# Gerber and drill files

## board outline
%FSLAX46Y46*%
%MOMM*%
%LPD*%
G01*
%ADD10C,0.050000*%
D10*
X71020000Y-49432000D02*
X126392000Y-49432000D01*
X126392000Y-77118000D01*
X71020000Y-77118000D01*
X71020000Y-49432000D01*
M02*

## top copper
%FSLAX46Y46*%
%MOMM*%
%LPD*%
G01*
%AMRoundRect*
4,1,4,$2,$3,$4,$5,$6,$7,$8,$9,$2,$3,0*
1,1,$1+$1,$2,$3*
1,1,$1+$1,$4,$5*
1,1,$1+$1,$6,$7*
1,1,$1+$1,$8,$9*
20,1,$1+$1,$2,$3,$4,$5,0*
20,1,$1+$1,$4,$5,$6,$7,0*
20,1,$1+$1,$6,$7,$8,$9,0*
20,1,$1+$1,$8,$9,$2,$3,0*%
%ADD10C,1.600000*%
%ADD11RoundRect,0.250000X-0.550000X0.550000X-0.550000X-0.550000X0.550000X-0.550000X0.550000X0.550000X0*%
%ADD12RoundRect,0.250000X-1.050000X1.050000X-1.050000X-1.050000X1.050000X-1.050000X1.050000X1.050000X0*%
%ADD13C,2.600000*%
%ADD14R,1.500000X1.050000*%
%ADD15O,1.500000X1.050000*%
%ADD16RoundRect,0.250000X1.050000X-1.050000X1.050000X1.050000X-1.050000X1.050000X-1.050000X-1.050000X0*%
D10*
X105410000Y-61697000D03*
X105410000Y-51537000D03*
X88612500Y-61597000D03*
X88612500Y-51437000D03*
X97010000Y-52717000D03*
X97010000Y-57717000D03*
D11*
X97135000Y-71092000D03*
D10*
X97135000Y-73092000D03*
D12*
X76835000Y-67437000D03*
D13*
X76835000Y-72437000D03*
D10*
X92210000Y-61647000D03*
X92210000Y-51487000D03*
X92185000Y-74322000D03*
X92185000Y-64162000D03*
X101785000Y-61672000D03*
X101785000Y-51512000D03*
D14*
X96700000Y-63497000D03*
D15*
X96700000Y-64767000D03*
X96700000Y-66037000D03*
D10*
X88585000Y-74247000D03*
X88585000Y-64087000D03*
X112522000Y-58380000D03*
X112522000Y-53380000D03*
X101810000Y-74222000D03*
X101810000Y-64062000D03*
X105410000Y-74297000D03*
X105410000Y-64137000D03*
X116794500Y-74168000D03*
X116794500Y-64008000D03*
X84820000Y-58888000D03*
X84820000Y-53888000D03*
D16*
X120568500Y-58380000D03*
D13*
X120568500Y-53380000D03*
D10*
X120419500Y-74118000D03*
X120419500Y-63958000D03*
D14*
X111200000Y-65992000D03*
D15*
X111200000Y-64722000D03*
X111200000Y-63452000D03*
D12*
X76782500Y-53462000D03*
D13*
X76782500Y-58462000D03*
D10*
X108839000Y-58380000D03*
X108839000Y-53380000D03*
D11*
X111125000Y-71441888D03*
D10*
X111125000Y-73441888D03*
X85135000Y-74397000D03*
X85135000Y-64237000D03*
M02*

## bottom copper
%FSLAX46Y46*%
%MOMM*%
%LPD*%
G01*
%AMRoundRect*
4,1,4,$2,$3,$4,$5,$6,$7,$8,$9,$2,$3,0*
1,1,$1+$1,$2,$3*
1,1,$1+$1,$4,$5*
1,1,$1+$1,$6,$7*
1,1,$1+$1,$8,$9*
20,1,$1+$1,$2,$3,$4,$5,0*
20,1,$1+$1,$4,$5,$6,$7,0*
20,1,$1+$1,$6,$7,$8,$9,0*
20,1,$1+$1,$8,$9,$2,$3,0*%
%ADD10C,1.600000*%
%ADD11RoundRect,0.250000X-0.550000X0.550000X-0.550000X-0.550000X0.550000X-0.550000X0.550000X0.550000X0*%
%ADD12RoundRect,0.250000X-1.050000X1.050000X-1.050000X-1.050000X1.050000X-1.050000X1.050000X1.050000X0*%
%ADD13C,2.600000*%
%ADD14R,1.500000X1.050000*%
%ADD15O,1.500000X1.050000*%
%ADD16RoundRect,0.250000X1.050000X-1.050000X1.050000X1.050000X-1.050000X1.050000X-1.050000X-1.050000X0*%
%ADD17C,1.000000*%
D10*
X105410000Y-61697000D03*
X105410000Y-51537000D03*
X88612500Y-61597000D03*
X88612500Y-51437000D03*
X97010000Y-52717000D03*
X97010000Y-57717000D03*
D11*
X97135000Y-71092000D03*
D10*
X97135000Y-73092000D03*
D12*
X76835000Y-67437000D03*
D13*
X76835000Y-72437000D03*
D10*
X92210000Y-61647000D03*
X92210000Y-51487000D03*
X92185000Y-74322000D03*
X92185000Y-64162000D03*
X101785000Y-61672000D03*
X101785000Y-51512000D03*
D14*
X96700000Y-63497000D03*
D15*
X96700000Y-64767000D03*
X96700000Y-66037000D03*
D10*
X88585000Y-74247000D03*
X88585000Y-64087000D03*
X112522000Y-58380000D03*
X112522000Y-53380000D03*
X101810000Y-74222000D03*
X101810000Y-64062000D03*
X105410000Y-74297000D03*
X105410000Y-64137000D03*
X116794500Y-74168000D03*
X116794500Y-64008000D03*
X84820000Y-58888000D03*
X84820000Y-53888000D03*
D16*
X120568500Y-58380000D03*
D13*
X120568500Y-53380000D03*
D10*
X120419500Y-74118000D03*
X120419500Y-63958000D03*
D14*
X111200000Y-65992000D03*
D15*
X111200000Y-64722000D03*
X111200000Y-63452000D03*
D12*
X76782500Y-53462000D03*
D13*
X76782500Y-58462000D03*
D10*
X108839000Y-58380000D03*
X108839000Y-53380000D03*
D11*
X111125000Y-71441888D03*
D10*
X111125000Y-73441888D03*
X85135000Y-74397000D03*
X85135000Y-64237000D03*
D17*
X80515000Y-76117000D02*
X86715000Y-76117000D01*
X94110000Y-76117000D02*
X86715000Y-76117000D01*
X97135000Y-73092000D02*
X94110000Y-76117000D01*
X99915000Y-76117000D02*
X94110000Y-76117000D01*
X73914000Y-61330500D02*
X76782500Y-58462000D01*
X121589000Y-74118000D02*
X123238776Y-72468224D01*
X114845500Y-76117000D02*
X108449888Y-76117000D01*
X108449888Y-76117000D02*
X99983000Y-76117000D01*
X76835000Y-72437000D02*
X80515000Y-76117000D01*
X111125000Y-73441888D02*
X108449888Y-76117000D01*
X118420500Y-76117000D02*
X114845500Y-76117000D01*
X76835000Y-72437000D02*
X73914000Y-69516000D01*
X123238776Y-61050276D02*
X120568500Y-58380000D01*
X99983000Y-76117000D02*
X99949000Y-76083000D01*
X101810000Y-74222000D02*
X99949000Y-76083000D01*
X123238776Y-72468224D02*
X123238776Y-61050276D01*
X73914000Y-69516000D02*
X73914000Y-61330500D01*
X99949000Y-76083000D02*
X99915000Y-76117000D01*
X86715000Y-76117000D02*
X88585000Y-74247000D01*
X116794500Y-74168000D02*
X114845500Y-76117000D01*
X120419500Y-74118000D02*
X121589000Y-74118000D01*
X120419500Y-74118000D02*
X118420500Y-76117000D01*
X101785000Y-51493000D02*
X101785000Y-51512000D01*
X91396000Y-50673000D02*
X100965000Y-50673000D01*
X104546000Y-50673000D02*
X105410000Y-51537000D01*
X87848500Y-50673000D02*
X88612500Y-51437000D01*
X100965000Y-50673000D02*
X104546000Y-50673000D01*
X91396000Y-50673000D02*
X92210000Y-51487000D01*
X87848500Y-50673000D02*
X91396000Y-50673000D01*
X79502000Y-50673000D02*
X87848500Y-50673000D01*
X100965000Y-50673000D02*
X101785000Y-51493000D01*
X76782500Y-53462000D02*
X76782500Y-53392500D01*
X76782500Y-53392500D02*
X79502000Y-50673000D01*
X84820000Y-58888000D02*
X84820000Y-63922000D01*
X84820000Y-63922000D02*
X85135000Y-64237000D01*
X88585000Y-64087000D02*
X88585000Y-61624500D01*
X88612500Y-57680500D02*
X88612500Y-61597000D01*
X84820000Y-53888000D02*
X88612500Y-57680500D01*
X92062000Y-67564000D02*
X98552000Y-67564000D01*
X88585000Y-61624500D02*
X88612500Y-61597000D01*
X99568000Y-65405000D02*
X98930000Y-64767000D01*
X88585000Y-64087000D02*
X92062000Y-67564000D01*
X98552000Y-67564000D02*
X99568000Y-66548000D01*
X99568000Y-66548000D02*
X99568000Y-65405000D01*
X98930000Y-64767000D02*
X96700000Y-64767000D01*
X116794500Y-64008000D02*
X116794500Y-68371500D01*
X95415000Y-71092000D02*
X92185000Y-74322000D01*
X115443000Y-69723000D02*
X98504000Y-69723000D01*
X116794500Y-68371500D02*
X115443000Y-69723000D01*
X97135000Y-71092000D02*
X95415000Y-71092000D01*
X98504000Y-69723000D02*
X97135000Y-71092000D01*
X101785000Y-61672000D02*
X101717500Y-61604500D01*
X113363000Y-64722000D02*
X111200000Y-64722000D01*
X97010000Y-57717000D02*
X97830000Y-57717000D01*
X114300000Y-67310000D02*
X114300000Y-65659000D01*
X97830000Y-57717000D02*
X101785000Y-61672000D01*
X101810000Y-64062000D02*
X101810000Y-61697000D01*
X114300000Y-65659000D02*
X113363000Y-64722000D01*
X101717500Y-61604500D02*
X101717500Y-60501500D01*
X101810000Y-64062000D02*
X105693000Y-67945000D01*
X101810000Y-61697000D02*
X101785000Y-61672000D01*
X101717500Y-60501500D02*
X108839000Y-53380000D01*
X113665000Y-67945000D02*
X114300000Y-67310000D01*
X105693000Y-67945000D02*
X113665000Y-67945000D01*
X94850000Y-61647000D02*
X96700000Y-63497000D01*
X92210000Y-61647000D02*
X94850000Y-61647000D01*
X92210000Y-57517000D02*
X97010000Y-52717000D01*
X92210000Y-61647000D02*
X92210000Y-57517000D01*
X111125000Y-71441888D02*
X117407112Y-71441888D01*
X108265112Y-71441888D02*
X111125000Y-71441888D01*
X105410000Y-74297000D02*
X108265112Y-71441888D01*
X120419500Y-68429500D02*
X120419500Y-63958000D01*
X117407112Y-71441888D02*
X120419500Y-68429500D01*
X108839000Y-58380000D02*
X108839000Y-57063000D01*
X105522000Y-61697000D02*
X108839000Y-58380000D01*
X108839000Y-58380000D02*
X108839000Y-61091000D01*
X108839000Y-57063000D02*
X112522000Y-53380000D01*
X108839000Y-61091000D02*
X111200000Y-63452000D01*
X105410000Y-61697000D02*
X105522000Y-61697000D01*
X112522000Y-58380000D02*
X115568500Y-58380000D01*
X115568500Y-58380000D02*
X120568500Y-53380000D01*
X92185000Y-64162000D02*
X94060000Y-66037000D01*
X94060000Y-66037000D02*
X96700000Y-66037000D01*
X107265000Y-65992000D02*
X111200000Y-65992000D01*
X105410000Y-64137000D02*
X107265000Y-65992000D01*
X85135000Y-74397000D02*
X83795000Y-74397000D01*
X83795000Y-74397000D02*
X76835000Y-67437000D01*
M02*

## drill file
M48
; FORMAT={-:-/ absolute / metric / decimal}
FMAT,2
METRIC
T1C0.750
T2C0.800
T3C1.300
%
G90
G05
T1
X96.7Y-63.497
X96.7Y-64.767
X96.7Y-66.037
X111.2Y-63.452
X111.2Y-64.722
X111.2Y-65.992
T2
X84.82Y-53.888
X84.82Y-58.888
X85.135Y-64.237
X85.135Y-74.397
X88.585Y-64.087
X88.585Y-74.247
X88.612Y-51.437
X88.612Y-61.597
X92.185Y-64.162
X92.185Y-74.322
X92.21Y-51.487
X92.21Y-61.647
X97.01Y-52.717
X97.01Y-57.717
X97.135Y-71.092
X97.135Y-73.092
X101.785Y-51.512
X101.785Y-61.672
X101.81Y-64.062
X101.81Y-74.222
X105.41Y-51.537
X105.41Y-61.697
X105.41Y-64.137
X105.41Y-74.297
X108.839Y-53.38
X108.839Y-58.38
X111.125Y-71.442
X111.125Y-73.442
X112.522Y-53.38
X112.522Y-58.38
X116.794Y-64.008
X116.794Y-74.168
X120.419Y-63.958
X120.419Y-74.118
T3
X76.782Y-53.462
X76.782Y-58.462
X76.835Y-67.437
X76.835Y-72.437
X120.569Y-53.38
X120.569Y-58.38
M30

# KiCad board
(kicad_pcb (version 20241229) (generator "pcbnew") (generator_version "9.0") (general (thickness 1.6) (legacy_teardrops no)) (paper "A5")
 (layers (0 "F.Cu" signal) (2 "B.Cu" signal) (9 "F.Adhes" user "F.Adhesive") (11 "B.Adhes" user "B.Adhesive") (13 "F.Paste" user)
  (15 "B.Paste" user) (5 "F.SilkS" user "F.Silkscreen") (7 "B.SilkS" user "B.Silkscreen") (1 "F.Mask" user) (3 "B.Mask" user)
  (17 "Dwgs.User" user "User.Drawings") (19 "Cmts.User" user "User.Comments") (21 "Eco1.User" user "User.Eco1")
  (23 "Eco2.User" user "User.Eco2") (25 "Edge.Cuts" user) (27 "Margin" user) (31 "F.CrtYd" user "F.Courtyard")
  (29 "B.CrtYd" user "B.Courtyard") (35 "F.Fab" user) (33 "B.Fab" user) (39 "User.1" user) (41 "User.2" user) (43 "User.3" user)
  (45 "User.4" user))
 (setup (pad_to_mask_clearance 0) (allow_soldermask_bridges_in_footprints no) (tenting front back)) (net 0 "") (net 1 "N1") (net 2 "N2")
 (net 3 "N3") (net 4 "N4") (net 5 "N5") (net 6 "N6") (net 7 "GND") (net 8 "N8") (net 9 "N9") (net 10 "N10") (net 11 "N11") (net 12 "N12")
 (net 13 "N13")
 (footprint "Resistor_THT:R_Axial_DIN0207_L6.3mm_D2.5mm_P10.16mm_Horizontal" (layer "F.Cu") (at 105.41 61.697 90)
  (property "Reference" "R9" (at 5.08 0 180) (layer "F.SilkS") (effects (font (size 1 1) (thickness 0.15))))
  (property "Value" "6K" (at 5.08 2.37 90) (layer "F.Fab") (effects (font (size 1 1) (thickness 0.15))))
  (pad "1" thru_hole circle (at 0 0 90) (size 1.6 1.6) (drill 0.8) (layers "*.Cu" "*.Mask") (remove_unused_layers no) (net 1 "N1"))
  (pad "2" thru_hole circle (at 10.16 0 90) (size 1.6 1.6) (drill 0.8) (layers "*.Cu" "*.Mask") (remove_unused_layers no) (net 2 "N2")))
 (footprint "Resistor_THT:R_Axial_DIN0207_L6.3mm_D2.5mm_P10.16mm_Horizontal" (layer "F.Cu") (at 88.6125 61.597 90)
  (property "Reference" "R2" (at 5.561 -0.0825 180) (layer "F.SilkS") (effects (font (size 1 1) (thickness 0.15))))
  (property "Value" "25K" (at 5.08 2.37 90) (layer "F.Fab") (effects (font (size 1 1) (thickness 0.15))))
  (pad "1" thru_hole circle (at 0 0 90) (size 1.6 1.6) (drill 0.8) (layers "*.Cu" "*.Mask") (remove_unused_layers no) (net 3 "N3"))
  (pad "2" thru_hole circle (at 10.16 0 90) (size 1.6 1.6) (drill 0.8) (layers "*.Cu" "*.Mask") (remove_unused_layers no) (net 2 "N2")))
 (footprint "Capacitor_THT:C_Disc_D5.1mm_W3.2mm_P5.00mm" (layer "F.Cu") (at 97.01 52.717 -90)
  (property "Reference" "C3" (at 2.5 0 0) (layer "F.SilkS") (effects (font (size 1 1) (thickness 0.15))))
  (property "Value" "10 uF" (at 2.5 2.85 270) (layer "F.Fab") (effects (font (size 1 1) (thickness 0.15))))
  (pad "1" thru_hole circle (at 0 0 270) (size 1.6 1.6) (drill 0.8) (layers "*.Cu" "*.Mask") (remove_unused_layers no) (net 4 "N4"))
  (pad "2" thru_hole circle (at 5 0 270) (size 1.6 1.6) (drill 0.8) (layers "*.Cu" "*.Mask") (remove_unused_layers no) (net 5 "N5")))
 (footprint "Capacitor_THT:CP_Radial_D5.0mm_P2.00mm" (layer "F.Cu") (at 97.135 71.092 -90)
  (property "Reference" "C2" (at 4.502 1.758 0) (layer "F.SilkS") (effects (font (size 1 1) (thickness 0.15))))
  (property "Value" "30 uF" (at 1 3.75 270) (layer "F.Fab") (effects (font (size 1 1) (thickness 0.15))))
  (pad "1" thru_hole roundrect (at 0 0 270) (size 1.6 1.6) (drill 0.8) (layers "*.Cu" "*.Mask") (remove_unused_layers no)
   (roundrect_rratio 0.15625) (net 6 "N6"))
  (pad "2" thru_hole circle (at 2 0 270) (size 1.6 1.6) (drill 0.8) (layers "*.Cu" "*.Mask") (remove_unused_layers no) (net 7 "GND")))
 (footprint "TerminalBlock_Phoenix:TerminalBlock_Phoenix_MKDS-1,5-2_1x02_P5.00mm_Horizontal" (layer "F.Cu") (at 76.835 67.437 -90)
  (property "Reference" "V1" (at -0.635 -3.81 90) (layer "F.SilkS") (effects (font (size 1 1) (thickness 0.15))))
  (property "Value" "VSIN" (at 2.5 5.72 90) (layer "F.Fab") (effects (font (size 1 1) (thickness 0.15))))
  (pad "1" thru_hole roundrect (at 0 0 270) (size 2.6 2.6) (drill 1.3) (layers "*.Cu" "*.Mask") (remove_unused_layers no)
   (roundrect_rratio 0.096154) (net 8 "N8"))
  (pad "2" thru_hole circle (at 5 0 270) (size 2.6 2.6) (drill 1.3) (layers "*.Cu" "*.Mask") (remove_unused_layers no) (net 7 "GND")))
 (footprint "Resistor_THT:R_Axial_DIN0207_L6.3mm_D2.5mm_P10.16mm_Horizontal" (layer "F.Cu") (at 92.21 61.647 90)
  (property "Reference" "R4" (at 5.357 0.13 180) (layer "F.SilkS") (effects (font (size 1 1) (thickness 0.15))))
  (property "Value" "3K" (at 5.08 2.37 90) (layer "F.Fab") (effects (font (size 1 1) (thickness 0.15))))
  (pad "1" thru_hole circle (at 0 0 90) (size 1.6 1.6) (drill 0.8) (layers "*.Cu" "*.Mask") (remove_unused_layers no) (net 4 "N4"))
  (pad "2" thru_hole circle (at 10.16 0 90) (size 1.6 1.6) (drill 0.8) (layers "*.Cu" "*.Mask") (remove_unused_layers no) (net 2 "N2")))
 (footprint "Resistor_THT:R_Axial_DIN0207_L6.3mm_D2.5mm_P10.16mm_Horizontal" (layer "F.Cu") (at 92.185 74.322 90)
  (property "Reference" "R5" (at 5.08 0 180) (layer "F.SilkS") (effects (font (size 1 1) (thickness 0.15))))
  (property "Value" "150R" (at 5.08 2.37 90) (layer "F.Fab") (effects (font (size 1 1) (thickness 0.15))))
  (pad "1" thru_hole circle (at 0 0 90) (size 1.6 1.6) (drill 0.8) (layers "*.Cu" "*.Mask") (remove_unused_layers no) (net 6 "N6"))
  (pad "2" thru_hole circle (at 10.16 0 90) (size 1.6 1.6) (drill 0.8) (layers "*.Cu" "*.Mask") (remove_unused_layers no) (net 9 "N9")))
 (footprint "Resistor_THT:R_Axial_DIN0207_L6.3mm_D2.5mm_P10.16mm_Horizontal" (layer "F.Cu") (at 101.785 61.672 90)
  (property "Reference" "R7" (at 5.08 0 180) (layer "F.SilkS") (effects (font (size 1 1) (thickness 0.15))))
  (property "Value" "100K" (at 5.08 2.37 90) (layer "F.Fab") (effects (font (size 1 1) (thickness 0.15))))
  (pad "1" thru_hole circle (at 0 0 90) (size 1.6 1.6) (drill 0.8) (layers "*.Cu" "*.Mask") (remove_unused_layers no) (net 5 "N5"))
  (pad "2" thru_hole circle (at 10.16 0 90) (size 1.6 1.6) (drill 0.8) (layers "*.Cu" "*.Mask") (remove_unused_layers no) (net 2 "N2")))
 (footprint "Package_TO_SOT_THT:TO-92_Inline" (layer "F.Cu") (at 96.7 63.497 -90)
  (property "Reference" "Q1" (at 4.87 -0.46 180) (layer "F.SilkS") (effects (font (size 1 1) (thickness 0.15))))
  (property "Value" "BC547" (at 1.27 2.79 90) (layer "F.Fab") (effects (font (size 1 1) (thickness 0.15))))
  (pad "1" thru_hole rect (at 0 0 270) (size 1.05 1.5) (drill 0.75) (layers "*.Cu" "*.Mask") (remove_unused_layers no) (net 4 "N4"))
  (pad "2" thru_hole oval (at 1.27 0 270) (size 1.05 1.5) (drill 0.75) (layers "*.Cu" "*.Mask") (remove_unused_layers no) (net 3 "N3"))
  (pad "3" thru_hole oval (at 2.54 0 270) (size 1.05 1.5) (drill 0.75) (layers "*.Cu" "*.Mask") (remove_unused_layers no) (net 9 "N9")))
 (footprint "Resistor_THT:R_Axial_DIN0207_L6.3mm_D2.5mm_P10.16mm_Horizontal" (layer "F.Cu") (at 88.585 74.247 90)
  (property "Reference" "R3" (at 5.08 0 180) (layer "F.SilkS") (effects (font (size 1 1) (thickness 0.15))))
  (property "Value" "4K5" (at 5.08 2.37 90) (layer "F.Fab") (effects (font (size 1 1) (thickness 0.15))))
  (pad "1" thru_hole circle (at 0 0 90) (size 1.6 1.6) (drill 0.8) (layers "*.Cu" "*.Mask") (remove_unused_layers no) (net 7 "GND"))
  (pad "2" thru_hole circle (at 10.16 0 90) (size 1.6 1.6) (drill 0.8) (layers "*.Cu" "*.Mask") (remove_unused_layers no) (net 3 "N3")))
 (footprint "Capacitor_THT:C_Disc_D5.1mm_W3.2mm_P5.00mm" (layer "F.Cu") (at 112.522 58.38 90)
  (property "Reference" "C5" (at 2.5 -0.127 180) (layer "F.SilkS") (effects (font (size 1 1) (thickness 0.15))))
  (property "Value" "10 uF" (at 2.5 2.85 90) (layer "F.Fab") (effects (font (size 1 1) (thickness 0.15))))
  (pad "1" thru_hole circle (at 0 0 90) (size 1.6 1.6) (drill 0.8) (layers "*.Cu" "*.Mask") (remove_unused_layers no) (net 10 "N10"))
  (pad "2" thru_hole circle (at 5 0 90) (size 1.6 1.6) (drill 0.8) (layers "*.Cu" "*.Mask") (remove_unused_layers no) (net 1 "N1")))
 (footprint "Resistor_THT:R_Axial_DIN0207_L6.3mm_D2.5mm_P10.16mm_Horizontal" (layer "F.Cu") (at 101.81 74.222 90)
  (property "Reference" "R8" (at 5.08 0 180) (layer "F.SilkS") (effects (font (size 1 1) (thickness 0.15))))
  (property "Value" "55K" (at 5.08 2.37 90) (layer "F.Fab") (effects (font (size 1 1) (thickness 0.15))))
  (pad "1" thru_hole circle (at 0 0 90) (size 1.6 1.6) (drill 0.8) (layers "*.Cu" "*.Mask") (remove_unused_layers no) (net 7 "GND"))
  (pad "2" thru_hole circle (at 10.16 0 90) (size 1.6 1.6) (drill 0.8) (layers "*.Cu" "*.Mask") (remove_unused_layers no) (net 5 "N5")))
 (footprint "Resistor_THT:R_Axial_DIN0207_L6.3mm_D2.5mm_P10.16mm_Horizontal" (layer "F.Cu") (at 105.41 74.297 90)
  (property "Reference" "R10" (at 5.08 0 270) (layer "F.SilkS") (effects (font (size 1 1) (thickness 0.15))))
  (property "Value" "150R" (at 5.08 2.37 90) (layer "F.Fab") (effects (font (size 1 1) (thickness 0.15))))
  (pad "1" thru_hole circle (at 0 0 90) (size 1.6 1.6) (drill 0.8) (layers "*.Cu" "*.Mask") (remove_unused_layers no) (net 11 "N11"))
  (pad "2" thru_hole circle (at 10.16 0 90) (size 1.6 1.6) (drill 0.8) (layers "*.Cu" "*.Mask") (remove_unused_layers no) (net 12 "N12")))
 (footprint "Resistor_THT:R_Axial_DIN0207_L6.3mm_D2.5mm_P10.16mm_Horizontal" (layer "F.Cu") (at 116.7945 74.168 90)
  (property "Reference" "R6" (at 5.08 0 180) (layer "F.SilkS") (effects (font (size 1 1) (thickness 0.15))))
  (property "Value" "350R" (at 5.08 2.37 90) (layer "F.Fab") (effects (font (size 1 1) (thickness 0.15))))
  (pad "1" thru_hole circle (at 0 0 90) (size 1.6 1.6) (drill 0.8) (layers "*.Cu" "*.Mask") (remove_unused_layers no) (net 7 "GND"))
  (pad "2" thru_hole circle (at 10.16 0 90) (size 1.6 1.6) (drill 0.8) (layers "*.Cu" "*.Mask") (remove_unused_layers no) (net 6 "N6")))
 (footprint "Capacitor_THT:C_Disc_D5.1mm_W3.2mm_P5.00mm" (layer "F.Cu") (at 84.82 58.888 90)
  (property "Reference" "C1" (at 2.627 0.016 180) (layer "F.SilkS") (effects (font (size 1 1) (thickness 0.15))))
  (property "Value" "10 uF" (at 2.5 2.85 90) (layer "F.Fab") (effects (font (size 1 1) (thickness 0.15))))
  (pad "1" thru_hole circle (at 0 0 90) (size 1.6 1.6) (drill 0.8) (layers "*.Cu" "*.Mask") (remove_unused_layers no) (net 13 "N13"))
  (pad "2" thru_hole circle (at 5 0 90) (size 1.6 1.6) (drill 0.8) (layers "*.Cu" "*.Mask") (remove_unused_layers no) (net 3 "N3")))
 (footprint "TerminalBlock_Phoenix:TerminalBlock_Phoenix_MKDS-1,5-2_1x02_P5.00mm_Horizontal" (layer "F.Cu") (at 120.5685 58.38 90)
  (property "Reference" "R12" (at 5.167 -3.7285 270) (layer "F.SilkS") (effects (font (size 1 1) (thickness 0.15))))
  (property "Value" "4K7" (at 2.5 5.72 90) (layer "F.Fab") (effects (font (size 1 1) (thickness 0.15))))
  (pad "1" thru_hole roundrect (at 0 0 90) (size 2.6 2.6) (drill 1.3) (layers "*.Cu" "*.Mask") (remove_unused_layers no)
   (roundrect_rratio 0.096154) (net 7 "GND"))
  (pad "2" thru_hole circle (at 5 0 90) (size 2.6 2.6) (drill 1.3) (layers "*.Cu" "*.Mask") (remove_unused_layers no) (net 10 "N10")))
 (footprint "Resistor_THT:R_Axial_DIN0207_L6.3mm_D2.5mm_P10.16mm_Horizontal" (layer "F.Cu") (at 120.4195 74.118 90)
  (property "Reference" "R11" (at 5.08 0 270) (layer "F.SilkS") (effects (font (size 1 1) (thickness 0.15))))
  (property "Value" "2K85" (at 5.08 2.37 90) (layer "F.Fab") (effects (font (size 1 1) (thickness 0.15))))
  (pad "1" thru_hole circle (at 0 0 90) (size 1.6 1.6) (drill 0.8) (layers "*.Cu" "*.Mask") (remove_unused_layers no) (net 7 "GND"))
  (pad "2" thru_hole circle (at 10.16 0 90) (size 1.6 1.6) (drill 0.8) (layers "*.Cu" "*.Mask") (remove_unused_layers no) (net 11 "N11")))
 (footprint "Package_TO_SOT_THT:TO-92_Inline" (layer "F.Cu") (at 111.2 65.992 90)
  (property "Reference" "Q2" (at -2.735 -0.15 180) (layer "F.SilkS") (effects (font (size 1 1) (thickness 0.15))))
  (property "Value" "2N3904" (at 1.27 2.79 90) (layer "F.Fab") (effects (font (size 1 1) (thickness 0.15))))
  (pad "1" thru_hole rect (at 0 0 90) (size 1.05 1.5) (drill 0.75) (layers "*.Cu" "*.Mask") (remove_unused_layers no) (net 12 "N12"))
  (pad "2" thru_hole oval (at 1.27 0 90) (size 1.05 1.5) (drill 0.75) (layers "*.Cu" "*.Mask") (remove_unused_layers no) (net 5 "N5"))
  (pad "3" thru_hole oval (at 2.54 0 90) (size 1.05 1.5) (drill 0.75) (layers "*.Cu" "*.Mask") (remove_unused_layers no) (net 1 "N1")))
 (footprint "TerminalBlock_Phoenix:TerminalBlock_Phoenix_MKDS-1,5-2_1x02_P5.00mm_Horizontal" (layer "F.Cu") (at 76.7825 53.462 -90)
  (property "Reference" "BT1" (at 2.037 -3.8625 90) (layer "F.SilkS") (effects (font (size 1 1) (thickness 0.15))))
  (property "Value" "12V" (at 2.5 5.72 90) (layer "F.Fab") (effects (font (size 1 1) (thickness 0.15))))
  (pad "1" thru_hole roundrect (at 0 0 270) (size 2.6 2.6) (drill 1.3) (layers "*.Cu" "*.Mask") (remove_unused_layers no)
   (roundrect_rratio 0.096154) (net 2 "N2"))
  (pad "2" thru_hole circle (at 5 0 270) (size 2.6 2.6) (drill 1.3) (layers "*.Cu" "*.Mask") (remove_unused_layers no) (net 7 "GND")))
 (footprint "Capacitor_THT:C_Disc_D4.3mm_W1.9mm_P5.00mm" (layer "F.Cu") (at 108.839 58.38 90)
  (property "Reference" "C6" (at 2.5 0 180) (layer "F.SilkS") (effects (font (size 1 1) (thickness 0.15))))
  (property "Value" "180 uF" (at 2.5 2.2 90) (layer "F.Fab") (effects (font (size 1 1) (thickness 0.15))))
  (pad "1" thru_hole circle (at 0 0 90) (size 1.6 1.6) (drill 0.8) (layers "*.Cu" "*.Mask") (remove_unused_layers no) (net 1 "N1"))
  (pad "2" thru_hole circle (at 5 0 90) (size 1.6 1.6) (drill 0.8) (layers "*.Cu" "*.Mask") (remove_unused_layers no) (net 5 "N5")))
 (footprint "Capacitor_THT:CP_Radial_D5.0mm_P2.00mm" (layer "F.Cu") (at 111.125 71.441888 -90)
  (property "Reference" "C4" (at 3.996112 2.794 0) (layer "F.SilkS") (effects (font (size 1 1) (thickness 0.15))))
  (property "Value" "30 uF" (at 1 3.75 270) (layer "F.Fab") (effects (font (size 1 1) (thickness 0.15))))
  (pad "1" thru_hole roundrect (at 0 0 270) (size 1.6 1.6) (drill 0.8) (layers "*.Cu" "*.Mask") (remove_unused_layers no)
   (roundrect_rratio 0.15625) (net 11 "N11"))
  (pad "2" thru_hole circle (at 2 0 270) (size 1.6 1.6) (drill 0.8) (layers "*.Cu" "*.Mask") (remove_unused_layers no) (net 7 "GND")))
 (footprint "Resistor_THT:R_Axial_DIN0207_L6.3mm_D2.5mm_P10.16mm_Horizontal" (layer "F.Cu") (at 85.135 74.397 90)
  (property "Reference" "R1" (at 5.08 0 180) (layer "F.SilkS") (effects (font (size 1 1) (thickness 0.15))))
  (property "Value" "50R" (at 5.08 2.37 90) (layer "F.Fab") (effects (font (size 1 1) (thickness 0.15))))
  (pad "1" thru_hole circle (at 0 0 90) (size 1.6 1.6) (drill 0.8) (layers "*.Cu" "*.Mask") (remove_unused_layers no) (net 8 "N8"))
  (pad "2" thru_hole circle (at 10.16 0 90) (size 1.6 1.6) (drill 0.8) (layers "*.Cu" "*.Mask") (remove_unused_layers no) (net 13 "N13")))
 (gr_rect (start 71.02 49.432) (end 126.392 77.118) (stroke (width 0.05) (type default)) (fill no) (layer "Edge.Cuts"))
 (segment (start 80.515 76.117) (end 86.715 76.117) (width 1) (layer "B.Cu") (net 7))
 (segment (start 94.11 76.117) (end 86.715 76.117) (width 1) (layer "B.Cu") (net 7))
 (segment (start 97.135 73.092) (end 94.11 76.117) (width 1) (layer "B.Cu") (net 7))
 (segment (start 99.915 76.117) (end 94.11 76.117) (width 1) (layer "B.Cu") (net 7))
 (segment (start 73.914 61.3305) (end 76.7825 58.462) (width 1) (layer "B.Cu") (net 7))
 (segment (start 121.589 74.118) (end 123.238776 72.468224) (width 1) (layer "B.Cu") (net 7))
 (segment (start 114.8455 76.117) (end 108.449888 76.117) (width 1) (layer "B.Cu") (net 7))
 (segment (start 108.449888 76.117) (end 99.983 76.117) (width 1) (layer "B.Cu") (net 7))
 (segment (start 76.835 72.437) (end 80.515 76.117) (width 1) (layer "B.Cu") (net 7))
 (segment (start 111.125 73.441888) (end 108.449888 76.117) (width 1) (layer "B.Cu") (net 7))
 (segment (start 118.4205 76.117) (end 114.8455 76.117) (width 1) (layer "B.Cu") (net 7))
 (segment (start 76.835 72.437) (end 73.914 69.516) (width 1) (layer "B.Cu") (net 7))
 (segment (start 123.238776 61.050276) (end 120.5685 58.38) (width 1) (layer "B.Cu") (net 7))
 (segment (start 99.983 76.117) (end 99.949 76.083) (width 1) (layer "B.Cu") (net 7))
 (segment (start 101.81 74.222) (end 99.949 76.083) (width 1) (layer "B.Cu") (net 7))
 (segment (start 123.238776 72.468224) (end 123.238776 61.050276) (width 1) (layer "B.Cu") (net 7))
 (segment (start 73.914 69.516) (end 73.914 61.3305) (width 1) (layer "B.Cu") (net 7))
 (segment (start 99.949 76.083) (end 99.915 76.117) (width 1) (layer "B.Cu") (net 7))
 (segment (start 86.715 76.117) (end 88.585 74.247) (width 1) (layer "B.Cu") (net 7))
 (segment (start 116.7945 74.168) (end 114.8455 76.117) (width 1) (layer "B.Cu") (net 7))
 (segment (start 120.4195 74.118) (end 121.589 74.118) (width 1) (layer "B.Cu") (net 7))
 (segment (start 120.4195 74.118) (end 118.4205 76.117) (width 1) (layer "B.Cu") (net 7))
 (segment (start 101.785 51.493) (end 101.785 51.512) (width 1) (layer "B.Cu") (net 2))
 (segment (start 91.396 50.673) (end 100.965 50.673) (width 1) (layer "B.Cu") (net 2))
 (segment (start 104.546 50.673) (end 105.41 51.537) (width 1) (layer "B.Cu") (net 2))
 (segment (start 87.8485 50.673) (end 88.6125 51.437) (width 1) (layer "B.Cu") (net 2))
 (segment (start 100.965 50.673) (end 104.546 50.673) (width 1) (layer "B.Cu") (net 2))
 (segment (start 91.396 50.673) (end 92.21 51.487) (width 1) (layer "B.Cu") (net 2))
 (segment (start 87.8485 50.673) (end 91.396 50.673) (width 1) (layer "B.Cu") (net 2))
 (segment (start 79.502 50.673) (end 87.8485 50.673) (width 1) (layer "B.Cu") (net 2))
 (segment (start 100.965 50.673) (end 101.785 51.493) (width 1) (layer "B.Cu") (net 2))
 (segment (start 76.7825 53.462) (end 76.7825 53.3925) (width 1) (layer "B.Cu") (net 2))
 (segment (start 76.7825 53.3925) (end 79.502 50.673) (width 1) (layer "B.Cu") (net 2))
 (segment (start 84.82 58.888) (end 84.82 63.922) (width 1) (layer "B.Cu") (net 13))
 (segment (start 84.82 63.922) (end 85.135 64.237) (width 1) (layer "B.Cu") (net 13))
 (segment (start 88.585 64.087) (end 88.585 61.6245) (width 1) (layer "B.Cu") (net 3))
 (segment (start 88.6125 57.6805) (end 88.6125 61.597) (width 1) (layer "B.Cu") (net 3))
 (segment (start 84.82 53.888) (end 88.6125 57.6805) (width 1) (layer "B.Cu") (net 3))
 (segment (start 92.062 67.564) (end 98.552 67.564) (width 1) (layer "B.Cu") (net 3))
 (segment (start 88.585 61.6245) (end 88.6125 61.597) (width 1) (layer "B.Cu") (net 3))
 (segment (start 99.568 65.405) (end 98.93 64.767) (width 1) (layer "B.Cu") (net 3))
 (segment (start 88.585 64.087) (end 92.062 67.564) (width 1) (layer "B.Cu") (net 3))
 (segment (start 98.552 67.564) (end 99.568 66.548) (width 1) (layer "B.Cu") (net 3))
 (segment (start 99.568 66.548) (end 99.568 65.405) (width 1) (layer "B.Cu") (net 3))
 (segment (start 98.93 64.767) (end 96.7 64.767) (width 1) (layer "B.Cu") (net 3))
 (segment (start 116.7945 64.008) (end 116.7945 68.3715) (width 1) (layer "B.Cu") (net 6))
 (segment (start 95.415 71.092) (end 92.185 74.322) (width 1) (layer "B.Cu") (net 6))
 (segment (start 115.443 69.723) (end 98.504 69.723) (width 1) (layer "B.Cu") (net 6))
 (segment (start 116.7945 68.3715) (end 115.443 69.723) (width 1) (layer "B.Cu") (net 6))
 (segment (start 97.135 71.092) (end 95.415 71.092) (width 1) (layer "B.Cu") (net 6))
 (segment (start 98.504 69.723) (end 97.135 71.092) (width 1) (layer "B.Cu") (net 6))
 (segment (start 101.785 61.672) (end 101.7175 61.6045) (width 1) (layer "B.Cu") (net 5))
 (segment (start 113.363 64.722) (end 111.2 64.722) (width 1) (layer "B.Cu") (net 5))
 (segment (start 97.01 57.717) (end 97.83 57.717) (width 1) (layer "B.Cu") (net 5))
 (segment (start 114.3 67.31) (end 114.3 65.659) (width 1) (layer "B.Cu") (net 5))
 (segment (start 97.83 57.717) (end 101.785 61.672) (width 1) (layer "B.Cu") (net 5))
 (segment (start 101.81 64.062) (end 101.81 61.697) (width 1) (layer "B.Cu") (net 5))
 (segment (start 114.3 65.659) (end 113.363 64.722) (width 1) (layer "B.Cu") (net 5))
 (segment (start 101.7175 61.6045) (end 101.7175 60.5015) (width 1) (layer "B.Cu") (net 5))
 (segment (start 101.81 64.062) (end 105.693 67.945) (width 1) (layer "B.Cu") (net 5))
 (segment (start 101.81 61.697) (end 101.785 61.672) (width 1) (layer "B.Cu") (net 5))
 (segment (start 101.7175 60.5015) (end 108.839 53.38) (width 1) (layer "B.Cu") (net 5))
 (segment (start 113.665 67.945) (end 114.3 67.31) (width 1) (layer "B.Cu") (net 5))
 (segment (start 105.693 67.945) (end 113.665 67.945) (width 1) (layer "B.Cu") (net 5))
 (segment (start 94.85 61.647) (end 96.7 63.497) (width 1) (layer "B.Cu") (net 4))
 (segment (start 92.21 61.647) (end 94.85 61.647) (width 1) (layer "B.Cu") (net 4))
 (segment (start 92.21 57.517) (end 97.01 52.717) (width 1) (layer "B.Cu") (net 4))
 (segment (start 92.21 61.647) (end 92.21 57.517) (width 1) (layer "B.Cu") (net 4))
 (segment (start 111.125 71.441888) (end 117.407112 71.441888) (width 1) (layer "B.Cu") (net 11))
 (segment (start 108.265112 71.441888) (end 111.125 71.441888) (width 1) (layer "B.Cu") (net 11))
 (segment (start 105.41 74.297) (end 108.265112 71.441888) (width 1) (layer "B.Cu") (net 11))
 (segment (start 120.4195 68.4295) (end 120.4195 63.958) (width 1) (layer "B.Cu") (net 11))
 (segment (start 117.407112 71.441888) (end 120.4195 68.4295) (width 1) (layer "B.Cu") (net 11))
 (segment (start 108.839 58.38) (end 108.839 57.063) (width 1) (layer "B.Cu") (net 1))
 (segment (start 105.522 61.697) (end 108.839 58.38) (width 1) (layer "B.Cu") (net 1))
 (segment (start 108.839 58.38) (end 108.839 61.091) (width 1) (layer "B.Cu") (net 1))
 (segment (start 108.839 57.063) (end 112.522 53.38) (width 1) (layer "B.Cu") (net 1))
 (segment (start 108.839 61.091) (end 111.2 63.452) (width 1) (layer "B.Cu") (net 1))
 (segment (start 105.41 61.697) (end 105.522 61.697) (width 1) (layer "B.Cu") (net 1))
 (segment (start 112.522 58.38) (end 115.5685 58.38) (width 1) (layer "B.Cu") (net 10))
 (segment (start 115.5685 58.38) (end 120.5685 53.38) (width 1) (layer "B.Cu") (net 10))
 (segment (start 92.185 64.162) (end 94.06 66.037) (width 1) (layer "B.Cu") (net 9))
 (segment (start 94.06 66.037) (end 96.7 66.037) (width 1) (layer "B.Cu") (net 9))
 (segment (start 107.265 65.992) (end 111.2 65.992) (width 1) (layer "B.Cu") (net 12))
 (segment (start 105.41 64.137) (end 107.265 65.992) (width 1) (layer "B.Cu") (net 12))
 (segment (start 85.135 74.397) (end 83.795 74.397) (width 1) (layer "B.Cu") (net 8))
 (segment (start 83.795 74.397) (end 76.835 67.437) (width 1) (layer "B.Cu") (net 8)))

